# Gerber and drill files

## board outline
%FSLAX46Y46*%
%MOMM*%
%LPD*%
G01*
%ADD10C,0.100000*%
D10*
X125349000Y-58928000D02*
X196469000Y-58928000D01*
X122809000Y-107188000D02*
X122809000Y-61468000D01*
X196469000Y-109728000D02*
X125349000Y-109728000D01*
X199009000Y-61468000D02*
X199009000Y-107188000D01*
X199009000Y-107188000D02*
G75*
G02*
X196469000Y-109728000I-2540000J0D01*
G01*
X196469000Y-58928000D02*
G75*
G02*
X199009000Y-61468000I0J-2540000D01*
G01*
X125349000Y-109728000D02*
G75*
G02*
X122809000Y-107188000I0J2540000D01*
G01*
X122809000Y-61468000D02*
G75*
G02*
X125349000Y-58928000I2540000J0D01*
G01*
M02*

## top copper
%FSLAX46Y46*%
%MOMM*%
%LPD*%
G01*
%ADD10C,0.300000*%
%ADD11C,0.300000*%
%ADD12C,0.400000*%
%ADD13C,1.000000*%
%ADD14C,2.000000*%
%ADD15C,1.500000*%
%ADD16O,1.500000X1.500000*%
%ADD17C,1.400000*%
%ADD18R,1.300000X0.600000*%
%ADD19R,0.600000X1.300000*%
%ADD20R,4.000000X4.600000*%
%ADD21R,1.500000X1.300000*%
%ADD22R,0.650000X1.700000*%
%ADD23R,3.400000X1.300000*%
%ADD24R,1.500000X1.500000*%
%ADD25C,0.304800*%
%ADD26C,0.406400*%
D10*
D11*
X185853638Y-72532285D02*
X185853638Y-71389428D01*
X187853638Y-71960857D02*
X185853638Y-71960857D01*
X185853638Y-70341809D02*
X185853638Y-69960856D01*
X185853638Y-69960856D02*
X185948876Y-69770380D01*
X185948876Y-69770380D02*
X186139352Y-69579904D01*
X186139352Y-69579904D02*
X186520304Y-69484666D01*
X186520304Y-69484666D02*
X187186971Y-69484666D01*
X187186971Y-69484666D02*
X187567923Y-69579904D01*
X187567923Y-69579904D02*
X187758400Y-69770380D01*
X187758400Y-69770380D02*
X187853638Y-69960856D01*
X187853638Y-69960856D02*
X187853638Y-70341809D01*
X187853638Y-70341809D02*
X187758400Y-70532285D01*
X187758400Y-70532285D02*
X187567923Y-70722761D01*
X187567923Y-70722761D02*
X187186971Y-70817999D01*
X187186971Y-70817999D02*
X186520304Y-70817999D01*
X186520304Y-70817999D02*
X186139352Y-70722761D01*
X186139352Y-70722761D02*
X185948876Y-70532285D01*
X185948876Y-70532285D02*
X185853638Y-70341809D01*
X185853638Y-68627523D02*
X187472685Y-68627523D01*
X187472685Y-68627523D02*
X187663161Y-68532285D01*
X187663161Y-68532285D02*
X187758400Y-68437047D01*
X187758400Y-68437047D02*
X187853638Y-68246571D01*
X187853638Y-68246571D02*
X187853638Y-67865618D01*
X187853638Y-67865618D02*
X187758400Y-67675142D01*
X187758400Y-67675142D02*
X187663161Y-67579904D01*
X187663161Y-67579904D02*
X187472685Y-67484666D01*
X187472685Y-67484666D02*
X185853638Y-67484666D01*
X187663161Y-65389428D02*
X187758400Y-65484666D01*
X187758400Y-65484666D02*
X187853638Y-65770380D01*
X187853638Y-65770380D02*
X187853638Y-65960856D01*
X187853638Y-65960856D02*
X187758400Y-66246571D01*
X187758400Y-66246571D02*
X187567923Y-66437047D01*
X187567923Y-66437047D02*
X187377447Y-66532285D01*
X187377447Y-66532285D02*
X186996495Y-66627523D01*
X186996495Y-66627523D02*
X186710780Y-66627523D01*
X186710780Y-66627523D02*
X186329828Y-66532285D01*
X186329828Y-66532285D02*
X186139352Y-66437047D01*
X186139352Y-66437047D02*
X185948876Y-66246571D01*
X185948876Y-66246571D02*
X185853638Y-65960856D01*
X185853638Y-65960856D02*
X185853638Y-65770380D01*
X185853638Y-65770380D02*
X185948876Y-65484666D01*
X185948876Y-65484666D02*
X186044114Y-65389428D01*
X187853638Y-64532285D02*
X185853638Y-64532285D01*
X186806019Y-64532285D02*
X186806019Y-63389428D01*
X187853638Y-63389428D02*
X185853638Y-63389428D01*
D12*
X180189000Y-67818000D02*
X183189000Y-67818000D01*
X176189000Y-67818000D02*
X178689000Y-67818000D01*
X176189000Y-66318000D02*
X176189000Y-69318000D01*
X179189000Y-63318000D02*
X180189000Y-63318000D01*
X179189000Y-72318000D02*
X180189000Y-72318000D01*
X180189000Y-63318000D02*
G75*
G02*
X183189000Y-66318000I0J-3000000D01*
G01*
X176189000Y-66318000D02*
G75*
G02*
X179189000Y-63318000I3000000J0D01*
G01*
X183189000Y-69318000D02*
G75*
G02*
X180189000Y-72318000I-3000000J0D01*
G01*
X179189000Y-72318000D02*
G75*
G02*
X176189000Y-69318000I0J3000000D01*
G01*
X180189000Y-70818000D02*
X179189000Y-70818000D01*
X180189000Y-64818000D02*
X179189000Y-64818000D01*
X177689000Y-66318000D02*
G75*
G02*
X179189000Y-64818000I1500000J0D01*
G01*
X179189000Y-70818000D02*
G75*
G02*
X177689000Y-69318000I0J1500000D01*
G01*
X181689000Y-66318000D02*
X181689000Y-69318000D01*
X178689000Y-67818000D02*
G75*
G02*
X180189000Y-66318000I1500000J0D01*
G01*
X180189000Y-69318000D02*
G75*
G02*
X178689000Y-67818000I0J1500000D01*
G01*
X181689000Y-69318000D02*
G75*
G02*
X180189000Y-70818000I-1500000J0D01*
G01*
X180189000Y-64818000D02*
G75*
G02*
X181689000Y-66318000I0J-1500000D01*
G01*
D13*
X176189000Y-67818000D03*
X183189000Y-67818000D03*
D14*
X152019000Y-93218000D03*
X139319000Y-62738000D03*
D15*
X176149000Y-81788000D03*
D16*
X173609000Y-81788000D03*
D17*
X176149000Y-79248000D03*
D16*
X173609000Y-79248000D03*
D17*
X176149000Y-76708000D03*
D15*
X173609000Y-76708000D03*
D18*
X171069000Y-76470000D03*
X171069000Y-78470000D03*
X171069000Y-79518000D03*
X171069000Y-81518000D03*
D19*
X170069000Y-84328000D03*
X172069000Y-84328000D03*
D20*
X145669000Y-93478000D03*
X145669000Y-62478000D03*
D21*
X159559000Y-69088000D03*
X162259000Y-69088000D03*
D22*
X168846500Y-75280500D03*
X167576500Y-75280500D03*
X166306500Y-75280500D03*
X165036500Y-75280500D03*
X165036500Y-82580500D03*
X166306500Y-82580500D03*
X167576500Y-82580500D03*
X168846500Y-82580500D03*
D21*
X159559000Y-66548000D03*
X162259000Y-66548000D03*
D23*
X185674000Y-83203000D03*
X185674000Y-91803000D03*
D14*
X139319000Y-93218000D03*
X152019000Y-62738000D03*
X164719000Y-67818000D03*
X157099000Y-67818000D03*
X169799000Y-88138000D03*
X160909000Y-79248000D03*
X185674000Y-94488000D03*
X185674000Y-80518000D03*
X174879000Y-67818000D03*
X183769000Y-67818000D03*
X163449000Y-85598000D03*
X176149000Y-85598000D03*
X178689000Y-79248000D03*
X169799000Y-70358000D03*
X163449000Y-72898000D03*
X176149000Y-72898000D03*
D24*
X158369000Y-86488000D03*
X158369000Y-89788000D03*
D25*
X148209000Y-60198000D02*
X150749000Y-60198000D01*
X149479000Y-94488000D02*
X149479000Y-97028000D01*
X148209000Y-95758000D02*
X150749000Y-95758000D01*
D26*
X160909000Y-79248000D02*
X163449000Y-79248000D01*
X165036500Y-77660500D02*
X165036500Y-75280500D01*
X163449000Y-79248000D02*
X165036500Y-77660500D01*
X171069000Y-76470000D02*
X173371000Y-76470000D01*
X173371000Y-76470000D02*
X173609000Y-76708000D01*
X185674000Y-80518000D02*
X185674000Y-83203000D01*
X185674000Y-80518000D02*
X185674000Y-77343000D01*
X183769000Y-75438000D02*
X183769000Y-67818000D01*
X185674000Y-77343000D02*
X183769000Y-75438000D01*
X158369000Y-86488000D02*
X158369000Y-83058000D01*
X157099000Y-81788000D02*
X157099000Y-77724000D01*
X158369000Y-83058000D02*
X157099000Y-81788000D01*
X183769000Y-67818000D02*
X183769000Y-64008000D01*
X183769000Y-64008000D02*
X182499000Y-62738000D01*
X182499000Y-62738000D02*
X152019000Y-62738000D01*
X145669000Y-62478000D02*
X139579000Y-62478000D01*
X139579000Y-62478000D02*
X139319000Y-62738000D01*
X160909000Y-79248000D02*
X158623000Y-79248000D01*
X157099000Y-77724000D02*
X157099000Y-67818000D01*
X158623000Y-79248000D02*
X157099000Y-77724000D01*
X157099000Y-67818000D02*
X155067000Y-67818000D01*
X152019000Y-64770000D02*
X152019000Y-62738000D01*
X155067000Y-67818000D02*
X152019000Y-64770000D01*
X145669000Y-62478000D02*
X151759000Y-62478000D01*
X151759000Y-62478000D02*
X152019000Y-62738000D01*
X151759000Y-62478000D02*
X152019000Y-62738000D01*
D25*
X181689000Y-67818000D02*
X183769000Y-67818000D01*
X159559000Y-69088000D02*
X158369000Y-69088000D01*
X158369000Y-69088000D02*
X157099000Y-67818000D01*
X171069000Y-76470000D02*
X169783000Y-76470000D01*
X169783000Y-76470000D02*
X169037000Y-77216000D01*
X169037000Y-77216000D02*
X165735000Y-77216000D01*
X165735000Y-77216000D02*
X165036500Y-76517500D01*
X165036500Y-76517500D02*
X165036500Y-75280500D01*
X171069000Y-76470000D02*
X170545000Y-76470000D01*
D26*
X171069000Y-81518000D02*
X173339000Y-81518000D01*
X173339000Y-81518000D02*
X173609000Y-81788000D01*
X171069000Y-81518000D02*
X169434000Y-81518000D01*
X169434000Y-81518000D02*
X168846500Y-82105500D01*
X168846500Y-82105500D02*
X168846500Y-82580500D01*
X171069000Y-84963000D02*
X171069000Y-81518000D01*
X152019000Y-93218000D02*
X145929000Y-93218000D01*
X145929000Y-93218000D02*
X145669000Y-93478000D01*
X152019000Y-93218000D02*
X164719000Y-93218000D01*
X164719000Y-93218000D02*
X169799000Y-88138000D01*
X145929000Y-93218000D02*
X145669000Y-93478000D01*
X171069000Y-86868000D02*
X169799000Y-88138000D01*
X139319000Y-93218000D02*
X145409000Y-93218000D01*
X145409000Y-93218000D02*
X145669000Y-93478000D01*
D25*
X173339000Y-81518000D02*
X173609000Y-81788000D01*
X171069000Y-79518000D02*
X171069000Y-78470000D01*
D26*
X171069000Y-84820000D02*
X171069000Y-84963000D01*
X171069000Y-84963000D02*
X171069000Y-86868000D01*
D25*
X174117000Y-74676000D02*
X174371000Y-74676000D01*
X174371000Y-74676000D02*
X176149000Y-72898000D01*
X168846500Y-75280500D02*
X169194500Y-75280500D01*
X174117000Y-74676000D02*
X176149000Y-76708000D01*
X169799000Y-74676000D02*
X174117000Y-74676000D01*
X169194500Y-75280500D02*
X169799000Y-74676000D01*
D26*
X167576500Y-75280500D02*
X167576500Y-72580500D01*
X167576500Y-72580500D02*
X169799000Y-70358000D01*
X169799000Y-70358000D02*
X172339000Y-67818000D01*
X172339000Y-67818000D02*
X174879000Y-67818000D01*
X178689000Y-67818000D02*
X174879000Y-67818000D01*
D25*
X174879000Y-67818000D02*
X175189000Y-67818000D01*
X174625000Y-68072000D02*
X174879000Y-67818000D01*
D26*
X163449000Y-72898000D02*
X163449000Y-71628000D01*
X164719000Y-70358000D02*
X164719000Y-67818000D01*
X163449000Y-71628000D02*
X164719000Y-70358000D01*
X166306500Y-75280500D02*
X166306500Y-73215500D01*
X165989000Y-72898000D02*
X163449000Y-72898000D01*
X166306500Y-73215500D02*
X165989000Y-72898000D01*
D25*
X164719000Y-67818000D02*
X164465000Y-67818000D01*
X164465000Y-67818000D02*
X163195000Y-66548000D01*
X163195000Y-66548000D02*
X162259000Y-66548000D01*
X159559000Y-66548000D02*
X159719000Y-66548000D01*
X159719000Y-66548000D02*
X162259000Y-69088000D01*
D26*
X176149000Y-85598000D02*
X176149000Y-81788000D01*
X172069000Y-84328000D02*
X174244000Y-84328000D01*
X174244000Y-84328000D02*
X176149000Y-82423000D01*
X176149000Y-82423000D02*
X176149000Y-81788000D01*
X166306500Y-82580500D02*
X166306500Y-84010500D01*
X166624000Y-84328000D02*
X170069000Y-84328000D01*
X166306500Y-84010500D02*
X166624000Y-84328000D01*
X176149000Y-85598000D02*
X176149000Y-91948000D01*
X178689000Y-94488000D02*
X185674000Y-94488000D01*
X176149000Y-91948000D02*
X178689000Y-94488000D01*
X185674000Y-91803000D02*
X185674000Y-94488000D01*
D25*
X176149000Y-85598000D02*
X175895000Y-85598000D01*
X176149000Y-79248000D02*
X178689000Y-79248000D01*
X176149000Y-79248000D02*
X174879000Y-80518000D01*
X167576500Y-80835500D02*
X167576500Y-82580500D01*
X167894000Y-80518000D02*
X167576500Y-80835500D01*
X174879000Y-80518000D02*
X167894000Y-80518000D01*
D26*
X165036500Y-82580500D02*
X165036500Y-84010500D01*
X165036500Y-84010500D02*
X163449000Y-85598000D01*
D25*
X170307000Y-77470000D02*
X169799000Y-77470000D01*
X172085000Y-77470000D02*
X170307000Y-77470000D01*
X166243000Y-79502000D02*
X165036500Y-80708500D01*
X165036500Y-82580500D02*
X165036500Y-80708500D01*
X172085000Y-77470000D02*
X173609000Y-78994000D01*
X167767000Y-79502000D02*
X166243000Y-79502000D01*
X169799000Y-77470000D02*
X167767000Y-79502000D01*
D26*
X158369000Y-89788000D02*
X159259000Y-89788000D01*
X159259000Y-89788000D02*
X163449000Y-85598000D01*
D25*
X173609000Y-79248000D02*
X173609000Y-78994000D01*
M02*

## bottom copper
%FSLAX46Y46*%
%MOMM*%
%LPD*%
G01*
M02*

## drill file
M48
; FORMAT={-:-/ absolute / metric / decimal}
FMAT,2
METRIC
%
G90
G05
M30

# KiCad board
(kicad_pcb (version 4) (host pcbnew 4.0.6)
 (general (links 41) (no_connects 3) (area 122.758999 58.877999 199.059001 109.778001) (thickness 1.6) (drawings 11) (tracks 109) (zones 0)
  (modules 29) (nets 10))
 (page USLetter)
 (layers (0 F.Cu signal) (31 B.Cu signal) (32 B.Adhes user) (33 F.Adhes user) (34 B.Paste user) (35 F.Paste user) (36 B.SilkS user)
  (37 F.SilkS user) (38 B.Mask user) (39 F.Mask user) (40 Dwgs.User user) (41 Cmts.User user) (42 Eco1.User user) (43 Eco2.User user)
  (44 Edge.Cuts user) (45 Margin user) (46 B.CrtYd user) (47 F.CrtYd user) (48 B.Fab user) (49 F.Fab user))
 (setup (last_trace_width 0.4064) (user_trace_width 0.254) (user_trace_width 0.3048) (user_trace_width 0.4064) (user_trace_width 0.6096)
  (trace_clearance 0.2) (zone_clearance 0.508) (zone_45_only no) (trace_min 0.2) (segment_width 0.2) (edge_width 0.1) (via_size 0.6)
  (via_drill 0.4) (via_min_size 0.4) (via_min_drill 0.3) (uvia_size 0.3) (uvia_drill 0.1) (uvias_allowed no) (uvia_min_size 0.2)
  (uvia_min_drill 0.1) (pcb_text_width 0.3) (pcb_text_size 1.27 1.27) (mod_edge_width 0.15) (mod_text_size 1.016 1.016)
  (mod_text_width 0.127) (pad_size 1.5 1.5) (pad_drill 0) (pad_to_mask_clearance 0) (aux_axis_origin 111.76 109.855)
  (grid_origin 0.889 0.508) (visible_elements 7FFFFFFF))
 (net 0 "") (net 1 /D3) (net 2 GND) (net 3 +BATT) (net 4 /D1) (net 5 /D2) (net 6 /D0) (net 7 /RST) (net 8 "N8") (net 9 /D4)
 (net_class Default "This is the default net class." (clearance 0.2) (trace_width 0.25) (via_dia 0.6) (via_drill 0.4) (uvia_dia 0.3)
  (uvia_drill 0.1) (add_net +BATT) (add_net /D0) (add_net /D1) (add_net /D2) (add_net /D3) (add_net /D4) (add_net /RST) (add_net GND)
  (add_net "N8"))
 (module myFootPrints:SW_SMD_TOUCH (layer F.Cu) (at 178.689 67.818 270)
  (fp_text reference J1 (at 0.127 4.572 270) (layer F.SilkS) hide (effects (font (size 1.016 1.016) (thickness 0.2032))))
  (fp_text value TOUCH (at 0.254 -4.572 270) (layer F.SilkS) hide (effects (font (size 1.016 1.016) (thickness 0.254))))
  (fp_line (start 0 -1.5) (end 0 -4.5) (layer F.Cu) (width 0.4)) (fp_line (start 0 2.5) (end 0 0) (layer F.Cu) (width 0.4))
  (fp_line (start -1.5 2.5) (end 1.5 2.5) (layer F.Cu) (width 0.4))
  (fp_line (start -4.5 -0.5) (end -4.5 -1.5) (layer F.Cu) (width 0.4))
  (fp_line (start 4.5 -0.5) (end 4.5 -1.5) (layer F.Cu) (width 0.4))
  (fp_arc (start -1.5 -1.5) (end -4.5 -1.5) (angle 90) (layer F.Cu) (width 0.4))
  (fp_arc (start -1.5 -0.5) (end -1.5 2.5) (angle 90) (layer F.Cu) (width 0.4))
  (fp_arc (start 1.5 -1.5) (end 1.5 -4.5) (angle 90) (layer F.Cu) (width 0.4))
  (fp_arc (start 1.5 -0.5) (end 4.5 -0.5) (angle 90) (layer F.Cu) (width 0.4))
  (fp_line (start 3 -1.5) (end 3 -0.5) (layer F.Cu) (width 0.4))
  (fp_line (start -3 -1.5) (end -3 -0.5) (layer F.Cu) (width 0.4))
  (fp_arc (start -1.5 -0.5) (end -1.5 1) (angle 90) (layer F.Cu) (width 0.4))
  (fp_arc (start 1.5 -0.5) (end 3 -0.5) (angle 90) (layer F.Cu) (width 0.4))
  (fp_line (start -1.5 -3) (end 1.5 -3) (layer F.Cu) (width 0.4))
  (fp_arc (start 0 -1.5) (end 0 0) (angle 90) (layer F.Cu) (width 0.4))
  (fp_arc (start 0 -1.5) (end 1.5 -1.5) (angle 90) (layer F.Cu) (width 0.4))
  (fp_arc (start 1.5 -1.5) (end 1.5 -3) (angle 90) (layer F.Cu) (width 0.4))
  (fp_arc (start -1.5 -1.5) (end -3 -1.5) (angle 90) (layer F.Cu) (width 0.4))
  (pad 2 smd circle (at 0 2.5 270) (size 1 1) (layers F.Cu) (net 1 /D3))
  (pad 1 smd circle (at 0 -4.5 270) (size 1 1) (layers F.Cu) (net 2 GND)))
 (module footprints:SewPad (layer F.Cu) (at 152.019 93.218)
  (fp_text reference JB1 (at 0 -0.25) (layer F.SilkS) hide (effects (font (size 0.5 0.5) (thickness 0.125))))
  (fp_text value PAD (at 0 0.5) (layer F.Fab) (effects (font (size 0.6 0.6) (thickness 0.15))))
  (pad 1 smd circle (at 0 0) (size 2 2) (layers F.Cu F.Mask) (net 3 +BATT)))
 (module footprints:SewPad (layer F.Cu) (at 139.319 62.738)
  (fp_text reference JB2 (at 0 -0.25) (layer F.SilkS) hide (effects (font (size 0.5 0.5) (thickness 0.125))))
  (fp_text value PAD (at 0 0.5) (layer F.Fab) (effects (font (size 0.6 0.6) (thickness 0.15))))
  (pad 1 smd circle (at 0 0) (size 2 2) (layers F.Cu F.Mask) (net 2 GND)))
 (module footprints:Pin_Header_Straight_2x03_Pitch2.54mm (layer F.Cu) (at 176.149 81.788 180)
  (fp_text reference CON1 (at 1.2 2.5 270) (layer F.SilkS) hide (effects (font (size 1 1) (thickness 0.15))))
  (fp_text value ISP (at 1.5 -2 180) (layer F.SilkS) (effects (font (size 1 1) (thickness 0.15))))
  (pad 1 smd circle (at 0 0 180) (size 1.5 1.5) (layers F.Cu) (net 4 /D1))
  (pad 2 smd oval (at 2.54 0 180) (size 1.5 1.5) (layers F.Cu) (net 3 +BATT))
  (pad 3 smd circle (at 0 2.54 180) (size 1.4 1.4) (layers F.Cu) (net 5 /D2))
  (pad 4 smd oval (at 2.54 2.54 180) (size 1.5 1.5) (layers F.Cu) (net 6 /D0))
  (pad 5 smd circle (at 0 5.08 180) (size 1.4 1.4) (layers F.Cu) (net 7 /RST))
  (pad 6 smd circle (at 2.54 5.08 180) (size 1.5 1.5) (layers F.Cu) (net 2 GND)))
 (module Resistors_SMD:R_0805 (layer F.Cu) (at 171.069 77.47 270)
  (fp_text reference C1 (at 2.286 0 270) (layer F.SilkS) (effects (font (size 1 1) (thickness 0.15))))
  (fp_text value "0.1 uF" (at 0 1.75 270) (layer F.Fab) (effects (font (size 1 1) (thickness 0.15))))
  (pad 1 smd rect (at -1 0 270) (size 0.6 1.3) (layers F.Cu F.Paste F.Mask) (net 2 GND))
  (pad 2 smd rect (at 1 0 270) (size 0.6 1.3) (layers F.Cu F.Paste F.Mask) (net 3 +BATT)))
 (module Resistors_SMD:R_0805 (layer F.Cu) (at 171.069 80.518 270)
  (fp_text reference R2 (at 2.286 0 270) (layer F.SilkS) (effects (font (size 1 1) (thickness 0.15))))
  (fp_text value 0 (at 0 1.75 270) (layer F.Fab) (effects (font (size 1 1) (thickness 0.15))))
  (pad 1 smd rect (at -1 0 270) (size 0.6 1.3) (layers F.Cu F.Paste F.Mask) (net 3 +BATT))
  (pad 2 smd rect (at 1 0 270) (size 0.6 1.3) (layers F.Cu F.Paste F.Mask) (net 3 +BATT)))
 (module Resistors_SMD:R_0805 (layer F.Cu) (at 171.069 84.328)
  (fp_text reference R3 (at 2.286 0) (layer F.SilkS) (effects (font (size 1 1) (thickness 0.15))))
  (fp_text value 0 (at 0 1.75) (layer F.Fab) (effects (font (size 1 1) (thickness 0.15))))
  (pad 1 smd rect (at -1 0) (size 0.6 1.3) (layers F.Cu F.Paste F.Mask) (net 4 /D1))
  (pad 2 smd rect (at 1 0) (size 0.6 1.3) (layers F.Cu F.Paste F.Mask) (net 4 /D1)))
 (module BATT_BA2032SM (layer F.Cu) (at 145.669 77.978 90)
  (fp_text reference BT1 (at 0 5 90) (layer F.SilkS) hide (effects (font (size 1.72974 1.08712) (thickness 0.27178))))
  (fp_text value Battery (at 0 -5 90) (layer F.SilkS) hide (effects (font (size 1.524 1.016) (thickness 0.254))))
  (pad 1 smd rect (at -15.5 0 90) (size 4.6 4) (layers F.Cu F.Paste F.Mask) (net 3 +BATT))
  (pad 2 smd rect (at 15.5 0 90) (size 4.6 4) (layers F.Cu F.Paste F.Mask) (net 2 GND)))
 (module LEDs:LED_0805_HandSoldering (layer F.Cu) (at 160.909 69.088)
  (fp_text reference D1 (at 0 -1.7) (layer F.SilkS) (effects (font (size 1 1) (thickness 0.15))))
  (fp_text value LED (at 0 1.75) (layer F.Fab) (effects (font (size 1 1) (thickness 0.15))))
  (pad 1 smd rect (at -1.35 0) (size 1.5 1.3) (layers F.Cu F.Paste F.Mask) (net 2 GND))
  (pad 2 smd rect (at 1.35 0) (size 1.5 1.3) (layers F.Cu F.Paste F.Mask) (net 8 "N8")))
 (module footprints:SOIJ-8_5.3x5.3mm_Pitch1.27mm (layer F.Cu) (at 166.9415 78.9305 270)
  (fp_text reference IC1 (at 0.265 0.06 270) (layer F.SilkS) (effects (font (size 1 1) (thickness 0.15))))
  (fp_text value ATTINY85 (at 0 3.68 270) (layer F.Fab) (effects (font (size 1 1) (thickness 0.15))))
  (pad 1 smd rect (at -3.65 -1.905 270) (size 1.7 0.65) (layers F.Cu F.Paste F.Mask) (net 7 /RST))
  (pad 2 smd rect (at -3.65 -0.635 270) (size 1.7 0.65) (layers F.Cu F.Paste F.Mask) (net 1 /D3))
  (pad 3 smd rect (at -3.65 0.635 270) (size 1.7 0.65) (layers F.Cu F.Paste F.Mask) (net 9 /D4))
  (pad 4 smd rect (at -3.65 1.905 270) (size 1.7 0.65) (layers F.Cu F.Paste F.Mask) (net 2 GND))
  (pad 5 smd rect (at 3.65 1.905 270) (size 1.7 0.65) (layers F.Cu F.Paste F.Mask) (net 6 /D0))
  (pad 6 smd rect (at 3.65 0.635 270) (size 1.7 0.65) (layers F.Cu F.Paste F.Mask) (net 4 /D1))
  (pad 7 smd rect (at 3.65 -0.635 270) (size 1.7 0.65) (layers F.Cu F.Paste F.Mask) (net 5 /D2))
  (pad 8 smd rect (at 3.65 -1.905 270) (size 1.7 0.65) (layers F.Cu F.Paste F.Mask) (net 3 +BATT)))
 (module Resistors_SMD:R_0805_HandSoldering (layer F.Cu) (at 160.909 66.548)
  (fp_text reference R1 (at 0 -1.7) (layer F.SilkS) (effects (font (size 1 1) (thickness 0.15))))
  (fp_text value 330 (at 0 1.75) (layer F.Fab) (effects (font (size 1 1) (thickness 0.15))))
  (pad 1 smd rect (at -1.35 0) (size 1.5 1.3) (layers F.Cu F.Paste F.Mask) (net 8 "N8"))
  (pad 2 smd rect (at 1.35 0) (size 1.5 1.3) (layers F.Cu F.Paste F.Mask) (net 9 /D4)))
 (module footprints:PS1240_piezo (layer F.Cu) (at 185.674 87.503 270)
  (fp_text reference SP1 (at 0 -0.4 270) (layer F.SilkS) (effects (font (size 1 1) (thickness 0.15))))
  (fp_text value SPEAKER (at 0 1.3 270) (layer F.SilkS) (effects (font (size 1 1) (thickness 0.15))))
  (pad 1 smd rect (at -4.3 0 270) (size 1.3 3.4) (layers F.Cu F.Paste F.Mask) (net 2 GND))
  (pad 2 smd rect (at 4.3 0 270) (size 1.3 3.4) (layers F.Cu F.Paste F.Mask) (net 4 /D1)))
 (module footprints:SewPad (layer F.Cu) (at 139.319 93.218)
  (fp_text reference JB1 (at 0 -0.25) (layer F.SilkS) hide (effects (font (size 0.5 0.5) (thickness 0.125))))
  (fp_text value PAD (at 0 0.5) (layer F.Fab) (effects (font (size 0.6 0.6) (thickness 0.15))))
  (pad 1 smd circle (at 0 0) (size 2 2) (layers F.Cu F.Mask) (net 3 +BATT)))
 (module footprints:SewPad (layer F.Cu) (at 152.019 62.738)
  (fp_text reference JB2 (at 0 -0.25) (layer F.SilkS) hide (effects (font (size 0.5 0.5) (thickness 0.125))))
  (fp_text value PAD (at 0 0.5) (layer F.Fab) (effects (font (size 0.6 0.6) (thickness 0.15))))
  (pad 1 smd circle (at 0 0) (size 2 2) (layers F.Cu F.Mask) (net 2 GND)))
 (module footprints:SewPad (layer F.Cu) (at 164.719 67.818)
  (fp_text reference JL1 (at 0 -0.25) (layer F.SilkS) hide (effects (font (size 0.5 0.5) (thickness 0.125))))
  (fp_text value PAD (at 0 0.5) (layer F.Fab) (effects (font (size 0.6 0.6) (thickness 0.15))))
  (pad 1 smd circle (at 0 0) (size 2 2) (layers F.Cu F.Mask) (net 9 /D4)))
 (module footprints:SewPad (layer F.Cu) (at 157.099 67.818)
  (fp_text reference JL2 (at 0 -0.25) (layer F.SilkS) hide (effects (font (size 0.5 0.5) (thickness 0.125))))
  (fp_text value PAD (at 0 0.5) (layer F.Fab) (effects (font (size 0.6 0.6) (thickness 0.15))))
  (pad 1 smd circle (at 0 0) (size 2 2) (layers F.Cu F.Mask) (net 2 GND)))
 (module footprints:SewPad (layer F.Cu) (at 169.799 88.138)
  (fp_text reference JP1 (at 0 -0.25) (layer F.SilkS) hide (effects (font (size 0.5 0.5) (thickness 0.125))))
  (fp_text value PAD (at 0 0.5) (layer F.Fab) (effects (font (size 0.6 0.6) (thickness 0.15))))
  (pad 1 smd circle (at 0 0) (size 2 2) (layers F.Cu F.Mask) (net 3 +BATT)))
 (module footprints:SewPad (layer F.Cu) (at 160.909 79.248)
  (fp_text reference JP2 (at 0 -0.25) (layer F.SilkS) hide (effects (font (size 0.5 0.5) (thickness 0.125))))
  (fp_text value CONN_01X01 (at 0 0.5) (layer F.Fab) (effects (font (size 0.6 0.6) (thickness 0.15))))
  (pad 1 smd circle (at 0 0) (size 2 2) (layers F.Cu F.Mask) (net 2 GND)))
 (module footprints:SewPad (layer F.Cu) (at 185.674 94.488)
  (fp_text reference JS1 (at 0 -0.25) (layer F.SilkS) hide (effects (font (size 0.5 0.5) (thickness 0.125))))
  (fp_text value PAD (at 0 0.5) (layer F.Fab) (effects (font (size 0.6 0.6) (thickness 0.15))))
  (pad 1 smd circle (at 0 0) (size 2 2) (layers F.Cu F.Mask) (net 4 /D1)))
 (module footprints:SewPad (layer F.Cu) (at 185.674 80.518)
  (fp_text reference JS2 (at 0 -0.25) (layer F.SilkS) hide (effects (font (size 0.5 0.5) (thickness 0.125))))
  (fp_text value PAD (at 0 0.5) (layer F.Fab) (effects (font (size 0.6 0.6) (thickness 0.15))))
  (pad 1 smd circle (at 0 0) (size 2 2) (layers F.Cu F.Mask) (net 2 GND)))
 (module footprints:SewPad (layer F.Cu) (at 174.879 67.818)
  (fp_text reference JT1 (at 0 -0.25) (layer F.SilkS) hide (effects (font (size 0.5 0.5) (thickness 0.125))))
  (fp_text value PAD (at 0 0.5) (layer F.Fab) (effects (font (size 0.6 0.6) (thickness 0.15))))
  (pad 1 smd circle (at 0 0) (size 2 2) (layers F.Cu F.Mask) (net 1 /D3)))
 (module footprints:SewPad (layer F.Cu) (at 183.769 67.818)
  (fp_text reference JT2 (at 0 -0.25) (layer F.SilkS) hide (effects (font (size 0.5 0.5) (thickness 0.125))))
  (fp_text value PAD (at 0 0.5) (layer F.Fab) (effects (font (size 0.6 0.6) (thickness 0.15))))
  (pad 1 smd circle (at 0 0) (size 2 2) (layers F.Cu F.Mask) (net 2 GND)))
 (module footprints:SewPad (layer F.Cu) (at 163.449 85.598)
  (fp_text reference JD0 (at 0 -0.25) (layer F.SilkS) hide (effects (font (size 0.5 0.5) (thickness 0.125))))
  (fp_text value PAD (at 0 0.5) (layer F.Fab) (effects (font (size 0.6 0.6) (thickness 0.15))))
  (pad 1 smd circle (at 0 0) (size 2 2) (layers F.Cu F.Mask) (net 6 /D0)))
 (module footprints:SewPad (layer F.Cu) (at 176.149 85.598)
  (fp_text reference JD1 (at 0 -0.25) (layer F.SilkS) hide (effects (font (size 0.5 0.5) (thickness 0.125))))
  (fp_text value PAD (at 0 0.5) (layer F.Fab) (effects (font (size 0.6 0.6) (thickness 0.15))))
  (pad 1 smd circle (at 0 0) (size 2 2) (layers F.Cu F.Mask) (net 4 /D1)))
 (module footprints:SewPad (layer F.Cu) (at 178.689 79.248)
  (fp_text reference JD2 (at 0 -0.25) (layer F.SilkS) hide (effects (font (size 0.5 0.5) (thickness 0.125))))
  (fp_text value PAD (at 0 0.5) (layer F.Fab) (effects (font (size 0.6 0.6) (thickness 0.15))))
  (pad 1 smd circle (at 0 0) (size 2 2) (layers F.Cu F.Mask) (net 5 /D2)))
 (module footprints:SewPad (layer F.Cu) (at 169.799 70.358)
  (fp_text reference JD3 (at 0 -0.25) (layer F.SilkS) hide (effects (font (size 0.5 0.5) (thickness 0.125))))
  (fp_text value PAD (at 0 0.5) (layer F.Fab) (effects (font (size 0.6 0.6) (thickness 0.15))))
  (pad 1 smd circle (at 0 0) (size 2 2) (layers F.Cu F.Mask) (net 1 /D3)))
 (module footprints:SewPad (layer F.Cu) (at 163.449 72.898)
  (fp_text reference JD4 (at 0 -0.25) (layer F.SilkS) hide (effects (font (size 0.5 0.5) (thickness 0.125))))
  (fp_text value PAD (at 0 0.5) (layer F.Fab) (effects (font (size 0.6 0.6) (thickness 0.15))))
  (pad 1 smd circle (at 0 0) (size 2 2) (layers F.Cu F.Mask) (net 9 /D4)))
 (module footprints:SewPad (layer F.Cu) (at 176.149 72.898)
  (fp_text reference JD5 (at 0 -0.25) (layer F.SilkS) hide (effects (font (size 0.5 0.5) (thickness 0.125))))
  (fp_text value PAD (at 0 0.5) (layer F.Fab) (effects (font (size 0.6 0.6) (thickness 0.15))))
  (pad 1 smd circle (at 0 0) (size 2 2) (layers F.Cu F.Mask) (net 7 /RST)))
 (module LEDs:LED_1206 (layer F.Cu) (at 158.369 88.138 90)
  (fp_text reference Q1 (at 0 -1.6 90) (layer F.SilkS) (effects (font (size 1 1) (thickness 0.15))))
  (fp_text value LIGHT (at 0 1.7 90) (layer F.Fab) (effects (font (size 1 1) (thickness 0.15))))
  (pad 2 smd rect (at 1.65 0 270) (size 1.5 1.5) (layers F.Cu F.Paste F.Mask) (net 2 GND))
  (pad 1 smd rect (at -1.65 0 270) (size 1.5 1.5) (layers F.Cu F.Paste F.Mask) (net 6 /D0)))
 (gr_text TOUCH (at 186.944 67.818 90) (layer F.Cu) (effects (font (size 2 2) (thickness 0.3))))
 (gr_line (start 125.349 58.928) (end 196.469 58.928) (angle 90) (layer Edge.Cuts) (width 0.1))
 (gr_line (start 122.809 107.188) (end 122.809 61.468) (angle 90) (layer Edge.Cuts) (width 0.1))
 (gr_line (start 196.469 109.728) (end 125.349 109.728) (angle 90) (layer Edge.Cuts) (width 0.1))
 (gr_line (start 199.009 61.468) (end 199.009 107.188) (angle 90) (layer Edge.Cuts) (width 0.1))
 (gr_arc (start 196.469 107.188) (end 199.009 107.188) (angle 90) (layer Edge.Cuts) (width 0.1))
 (gr_arc (start 196.469 61.468) (end 196.469 58.928) (angle 90) (layer Edge.Cuts) (width 0.1))
 (gr_arc (start 125.349 107.188) (end 125.349 109.728) (angle 90) (layer Edge.Cuts) (width 0.1))
 (gr_arc (start 125.349 61.468) (end 122.809 61.468) (angle 90) (layer Edge.Cuts) (width 0.1))
 (segment (start 148.209 60.198) (end 150.749 60.198) (width 0.3048) (layer F.Cu) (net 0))
 (segment (start 149.479 94.488) (end 149.479 97.028) (width 0.3048) (layer F.Cu) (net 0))
 (segment (start 148.209 95.758) (end 150.749 95.758) (width 0.3048) (layer F.Cu) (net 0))
 (segment (start 160.909 79.248) (end 163.449 79.248) (width 0.4064) (layer F.Cu) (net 2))
 (segment (start 165.0365 77.6605) (end 165.0365 75.2805) (width 0.4064) (layer F.Cu) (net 2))
 (segment (start 163.449 79.248) (end 165.0365 77.6605) (width 0.4064) (layer F.Cu) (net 2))
 (segment (start 171.069 76.47) (end 173.371 76.47) (width 0.4064) (layer F.Cu) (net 2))
 (segment (start 173.371 76.47) (end 173.609 76.708) (width 0.4064) (layer F.Cu) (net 2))
 (segment (start 185.674 80.518) (end 185.674 83.203) (width 0.4064) (layer F.Cu) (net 2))
 (segment (start 185.674 80.518) (end 185.674 77.343) (width 0.4064) (layer F.Cu) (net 2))
 (segment (start 183.769 75.438) (end 183.769 67.818) (width 0.4064) (layer F.Cu) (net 2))
 (segment (start 185.674 77.343) (end 183.769 75.438) (width 0.4064) (layer F.Cu) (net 2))
 (segment (start 158.369 86.488) (end 158.369 83.058) (width 0.4064) (layer F.Cu) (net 2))
 (segment (start 157.099 81.788) (end 157.099 77.724) (width 0.4064) (layer F.Cu) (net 2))
 (segment (start 158.369 83.058) (end 157.099 81.788) (width 0.4064) (layer F.Cu) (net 2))
 (segment (start 183.769 67.818) (end 183.769 64.008) (width 0.4064) (layer F.Cu) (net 2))
 (segment (start 183.769 64.008) (end 182.499 62.738) (width 0.4064) (layer F.Cu) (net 2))
 (segment (start 182.499 62.738) (end 152.019 62.738) (width 0.4064) (layer F.Cu) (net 2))
 (segment (start 145.669 62.478) (end 139.579 62.478) (width 0.4064) (layer F.Cu) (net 2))
 (segment (start 139.579 62.478) (end 139.319 62.738) (width 0.4064) (layer F.Cu) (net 2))
 (segment (start 160.909 79.248) (end 158.623 79.248) (width 0.4064) (layer F.Cu) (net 2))
 (segment (start 157.099 77.724) (end 157.099 67.818) (width 0.4064) (layer F.Cu) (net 2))
 (segment (start 158.623 79.248) (end 157.099 77.724) (width 0.4064) (layer F.Cu) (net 2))
 (segment (start 157.099 67.818) (end 155.067 67.818) (width 0.4064) (layer F.Cu) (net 2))
 (segment (start 152.019 64.77) (end 152.019 62.738) (width 0.4064) (layer F.Cu) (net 2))
 (segment (start 155.067 67.818) (end 152.019 64.77) (width 0.4064) (layer F.Cu) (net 2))
 (segment (start 145.669 62.478) (end 151.759 62.478) (width 0.4064) (layer F.Cu) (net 2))
 (segment (start 151.759 62.478) (end 152.019 62.738) (width 0.4064) (layer F.Cu) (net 2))
 (segment (start 151.759 62.478) (end 152.019 62.738) (width 0.4064) (layer F.Cu) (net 2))
 (segment (start 181.689 67.818) (end 183.769 67.818) (width 0.3048) (layer F.Cu) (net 2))
 (segment (start 159.559 69.088) (end 158.369 69.088) (width 0.3048) (layer F.Cu) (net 2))
 (segment (start 158.369 69.088) (end 157.099 67.818) (width 0.3048) (layer F.Cu) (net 2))
 (segment (start 171.069 76.47) (end 169.783 76.47) (width 0.3048) (layer F.Cu) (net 2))
 (segment (start 169.783 76.47) (end 169.037 77.216) (width 0.3048) (layer F.Cu) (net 2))
 (segment (start 169.037 77.216) (end 165.735 77.216) (width 0.3048) (layer F.Cu) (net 2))
 (segment (start 165.735 77.216) (end 165.0365 76.5175) (width 0.3048) (layer F.Cu) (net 2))
 (segment (start 165.0365 76.5175) (end 165.0365 75.2805) (width 0.3048) (layer F.Cu) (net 2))
 (segment (start 171.069 76.47) (end 170.545 76.47) (width 0.3048) (layer F.Cu) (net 2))
 (segment (start 171.069 81.518) (end 173.339 81.518) (width 0.4064) (layer F.Cu) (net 3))
 (segment (start 173.339 81.518) (end 173.609 81.788) (width 0.4064) (layer F.Cu) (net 3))
 (segment (start 171.069 81.518) (end 169.434 81.518) (width 0.4064) (layer F.Cu) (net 3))
 (segment (start 169.434 81.518) (end 168.8465 82.1055) (width 0.4064) (layer F.Cu) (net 3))
 (segment (start 168.8465 82.1055) (end 168.8465 82.5805) (width 0.4064) (layer F.Cu) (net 3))
 (segment (start 171.069 84.963) (end 171.069 81.518) (width 0.4064) (layer F.Cu) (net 3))
 (segment (start 152.019 93.218) (end 145.929 93.218) (width 0.4064) (layer F.Cu) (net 3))
 (segment (start 145.929 93.218) (end 145.669 93.478) (width 0.4064) (layer F.Cu) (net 3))
 (segment (start 152.019 93.218) (end 164.719 93.218) (width 0.4064) (layer F.Cu) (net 3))
 (segment (start 164.719 93.218) (end 169.799 88.138) (width 0.4064) (layer F.Cu) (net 3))
 (segment (start 145.929 93.218) (end 145.669 93.478) (width 0.4064) (layer F.Cu) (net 3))
 (segment (start 171.069 86.868) (end 169.799 88.138) (width 0.4064) (layer F.Cu) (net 3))
 (segment (start 139.319 93.218) (end 145.409 93.218) (width 0.4064) (layer F.Cu) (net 3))
 (segment (start 145.409 93.218) (end 145.669 93.478) (width 0.4064) (layer F.Cu) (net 3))
 (segment (start 173.339 81.518) (end 173.609 81.788) (width 0.3048) (layer F.Cu) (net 3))
 (segment (start 171.069 79.518) (end 171.069 78.47) (width 0.3048) (layer F.Cu) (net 3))
 (segment (start 171.069 84.82) (end 171.069 84.963) (width 0.4064) (layer F.Cu) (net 3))
 (segment (start 171.069 84.963) (end 171.069 86.868) (width 0.4064) (layer F.Cu) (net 3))
 (segment (start 174.117 74.676) (end 174.371 74.676) (width 0.3048) (layer F.Cu) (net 7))
 (segment (start 174.371 74.676) (end 176.149 72.898) (width 0.3048) (layer F.Cu) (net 7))
 (segment (start 168.8465 75.2805) (end 169.1945 75.2805) (width 0.3048) (layer F.Cu) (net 7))
 (segment (start 174.117 74.676) (end 176.149 76.708) (width 0.3048) (layer F.Cu) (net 7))
 (segment (start 169.799 74.676) (end 174.117 74.676) (width 0.3048) (layer F.Cu) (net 7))
 (segment (start 169.1945 75.2805) (end 169.799 74.676) (width 0.3048) (layer F.Cu) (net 7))
 (segment (start 167.5765 75.2805) (end 167.5765 72.5805) (width 0.4064) (layer F.Cu) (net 1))
 (segment (start 167.5765 72.5805) (end 169.799 70.358) (width 0.4064) (layer F.Cu) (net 1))
 (segment (start 169.799 70.358) (end 172.339 67.818) (width 0.4064) (layer F.Cu) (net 1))
 (segment (start 172.339 67.818) (end 174.879 67.818) (width 0.4064) (layer F.Cu) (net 1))
 (segment (start 178.689 67.818) (end 174.879 67.818) (width 0.4064) (layer F.Cu) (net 1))
 (segment (start 174.879 67.818) (end 175.189 67.818) (width 0.3048) (layer F.Cu) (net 1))
 (segment (start 174.625 68.072) (end 174.879 67.818) (width 0.3048) (layer F.Cu) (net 1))
 (segment (start 163.449 72.898) (end 163.449 71.628) (width 0.4064) (layer F.Cu) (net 9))
 (segment (start 164.719 70.358) (end 164.719 67.818) (width 0.4064) (layer F.Cu) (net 9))
 (segment (start 163.449 71.628) (end 164.719 70.358) (width 0.4064) (layer F.Cu) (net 9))
 (segment (start 166.3065 75.2805) (end 166.3065 73.2155) (width 0.4064) (layer F.Cu) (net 9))
 (segment (start 165.989 72.898) (end 163.449 72.898) (width 0.4064) (layer F.Cu) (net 9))
 (segment (start 166.3065 73.2155) (end 165.989 72.898) (width 0.4064) (layer F.Cu) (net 9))
 (segment (start 164.719 67.818) (end 164.465 67.818) (width 0.3048) (layer F.Cu) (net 9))
 (segment (start 164.465 67.818) (end 163.195 66.548) (width 0.3048) (layer F.Cu) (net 9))
 (segment (start 163.195 66.548) (end 162.259 66.548) (width 0.3048) (layer F.Cu) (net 9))
 (segment (start 159.559 66.548) (end 159.719 66.548) (width 0.3048) (layer F.Cu) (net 8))
 (segment (start 159.719 66.548) (end 162.259 69.088) (width 0.3048) (layer F.Cu) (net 8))
 (segment (start 176.149 85.598) (end 176.149 81.788) (width 0.4064) (layer F.Cu) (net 4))
 (segment (start 172.069 84.328) (end 174.244 84.328) (width 0.4064) (layer F.Cu) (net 4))
 (segment (start 174.244 84.328) (end 176.149 82.423) (width 0.4064) (layer F.Cu) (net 4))
 (segment (start 176.149 82.423) (end 176.149 81.788) (width 0.4064) (layer F.Cu) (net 4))
 (segment (start 166.3065 82.5805) (end 166.3065 84.0105) (width 0.4064) (layer F.Cu) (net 4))
 (segment (start 166.624 84.328) (end 170.069 84.328) (width 0.4064) (layer F.Cu) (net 4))
 (segment (start 166.3065 84.0105) (end 166.624 84.328) (width 0.4064) (layer F.Cu) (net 4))
 (segment (start 176.149 85.598) (end 176.149 91.948) (width 0.4064) (layer F.Cu) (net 4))
 (segment (start 178.689 94.488) (end 185.674 94.488) (width 0.4064) (layer F.Cu) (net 4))
 (segment (start 176.149 91.948) (end 178.689 94.488) (width 0.4064) (layer F.Cu) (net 4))
 (segment (start 185.674 91.803) (end 185.674 94.488) (width 0.4064) (layer F.Cu) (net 4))
 (segment (start 176.149 85.598) (end 175.895 85.598) (width 0.3048) (layer F.Cu) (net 4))
 (segment (start 176.149 79.248) (end 178.689 79.248) (width 0.3048) (layer F.Cu) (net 5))
 (segment (start 176.149 79.248) (end 174.879 80.518) (width 0.3048) (layer F.Cu) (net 5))
 (segment (start 167.5765 80.8355) (end 167.5765 82.5805) (width 0.3048) (layer F.Cu) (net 5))
 (segment (start 167.894 80.518) (end 167.5765 80.8355) (width 0.3048) (layer F.Cu) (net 5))
 (segment (start 174.879 80.518) (end 167.894 80.518) (width 0.3048) (layer F.Cu) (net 5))
 (segment (start 165.0365 82.5805) (end 165.0365 84.0105) (width 0.4064) (layer F.Cu) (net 6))
 (segment (start 165.0365 84.0105) (end 163.449 85.598) (width 0.4064) (layer F.Cu) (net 6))
 (segment (start 170.307 77.47) (end 169.799 77.47) (width 0.3048) (layer F.Cu) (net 6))
 (segment (start 172.085 77.47) (end 170.307 77.47) (width 0.3048) (layer F.Cu) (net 6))
 (segment (start 166.243 79.502) (end 165.0365 80.7085) (width 0.3048) (layer F.Cu) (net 6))
 (segment (start 165.0365 82.5805) (end 165.0365 80.7085) (width 0.3048) (layer F.Cu) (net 6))
 (segment (start 172.085 77.47) (end 173.609 78.994) (width 0.3048) (layer F.Cu) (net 6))
 (segment (start 167.767 79.502) (end 166.243 79.502) (width 0.3048) (layer F.Cu) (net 6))
 (segment (start 169.799 77.47) (end 167.767 79.502) (width 0.3048) (layer F.Cu) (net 6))
 (segment (start 158.369 89.788) (end 159.259 89.788) (width 0.4064) (layer F.Cu) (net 6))
 (segment (start 159.259 89.788) (end 163.449 85.598) (width 0.4064) (layer F.Cu) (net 6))
 (segment (start 173.609 79.248) (end 173.609 78.994) (width 0.3048) (layer F.Cu) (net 6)))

